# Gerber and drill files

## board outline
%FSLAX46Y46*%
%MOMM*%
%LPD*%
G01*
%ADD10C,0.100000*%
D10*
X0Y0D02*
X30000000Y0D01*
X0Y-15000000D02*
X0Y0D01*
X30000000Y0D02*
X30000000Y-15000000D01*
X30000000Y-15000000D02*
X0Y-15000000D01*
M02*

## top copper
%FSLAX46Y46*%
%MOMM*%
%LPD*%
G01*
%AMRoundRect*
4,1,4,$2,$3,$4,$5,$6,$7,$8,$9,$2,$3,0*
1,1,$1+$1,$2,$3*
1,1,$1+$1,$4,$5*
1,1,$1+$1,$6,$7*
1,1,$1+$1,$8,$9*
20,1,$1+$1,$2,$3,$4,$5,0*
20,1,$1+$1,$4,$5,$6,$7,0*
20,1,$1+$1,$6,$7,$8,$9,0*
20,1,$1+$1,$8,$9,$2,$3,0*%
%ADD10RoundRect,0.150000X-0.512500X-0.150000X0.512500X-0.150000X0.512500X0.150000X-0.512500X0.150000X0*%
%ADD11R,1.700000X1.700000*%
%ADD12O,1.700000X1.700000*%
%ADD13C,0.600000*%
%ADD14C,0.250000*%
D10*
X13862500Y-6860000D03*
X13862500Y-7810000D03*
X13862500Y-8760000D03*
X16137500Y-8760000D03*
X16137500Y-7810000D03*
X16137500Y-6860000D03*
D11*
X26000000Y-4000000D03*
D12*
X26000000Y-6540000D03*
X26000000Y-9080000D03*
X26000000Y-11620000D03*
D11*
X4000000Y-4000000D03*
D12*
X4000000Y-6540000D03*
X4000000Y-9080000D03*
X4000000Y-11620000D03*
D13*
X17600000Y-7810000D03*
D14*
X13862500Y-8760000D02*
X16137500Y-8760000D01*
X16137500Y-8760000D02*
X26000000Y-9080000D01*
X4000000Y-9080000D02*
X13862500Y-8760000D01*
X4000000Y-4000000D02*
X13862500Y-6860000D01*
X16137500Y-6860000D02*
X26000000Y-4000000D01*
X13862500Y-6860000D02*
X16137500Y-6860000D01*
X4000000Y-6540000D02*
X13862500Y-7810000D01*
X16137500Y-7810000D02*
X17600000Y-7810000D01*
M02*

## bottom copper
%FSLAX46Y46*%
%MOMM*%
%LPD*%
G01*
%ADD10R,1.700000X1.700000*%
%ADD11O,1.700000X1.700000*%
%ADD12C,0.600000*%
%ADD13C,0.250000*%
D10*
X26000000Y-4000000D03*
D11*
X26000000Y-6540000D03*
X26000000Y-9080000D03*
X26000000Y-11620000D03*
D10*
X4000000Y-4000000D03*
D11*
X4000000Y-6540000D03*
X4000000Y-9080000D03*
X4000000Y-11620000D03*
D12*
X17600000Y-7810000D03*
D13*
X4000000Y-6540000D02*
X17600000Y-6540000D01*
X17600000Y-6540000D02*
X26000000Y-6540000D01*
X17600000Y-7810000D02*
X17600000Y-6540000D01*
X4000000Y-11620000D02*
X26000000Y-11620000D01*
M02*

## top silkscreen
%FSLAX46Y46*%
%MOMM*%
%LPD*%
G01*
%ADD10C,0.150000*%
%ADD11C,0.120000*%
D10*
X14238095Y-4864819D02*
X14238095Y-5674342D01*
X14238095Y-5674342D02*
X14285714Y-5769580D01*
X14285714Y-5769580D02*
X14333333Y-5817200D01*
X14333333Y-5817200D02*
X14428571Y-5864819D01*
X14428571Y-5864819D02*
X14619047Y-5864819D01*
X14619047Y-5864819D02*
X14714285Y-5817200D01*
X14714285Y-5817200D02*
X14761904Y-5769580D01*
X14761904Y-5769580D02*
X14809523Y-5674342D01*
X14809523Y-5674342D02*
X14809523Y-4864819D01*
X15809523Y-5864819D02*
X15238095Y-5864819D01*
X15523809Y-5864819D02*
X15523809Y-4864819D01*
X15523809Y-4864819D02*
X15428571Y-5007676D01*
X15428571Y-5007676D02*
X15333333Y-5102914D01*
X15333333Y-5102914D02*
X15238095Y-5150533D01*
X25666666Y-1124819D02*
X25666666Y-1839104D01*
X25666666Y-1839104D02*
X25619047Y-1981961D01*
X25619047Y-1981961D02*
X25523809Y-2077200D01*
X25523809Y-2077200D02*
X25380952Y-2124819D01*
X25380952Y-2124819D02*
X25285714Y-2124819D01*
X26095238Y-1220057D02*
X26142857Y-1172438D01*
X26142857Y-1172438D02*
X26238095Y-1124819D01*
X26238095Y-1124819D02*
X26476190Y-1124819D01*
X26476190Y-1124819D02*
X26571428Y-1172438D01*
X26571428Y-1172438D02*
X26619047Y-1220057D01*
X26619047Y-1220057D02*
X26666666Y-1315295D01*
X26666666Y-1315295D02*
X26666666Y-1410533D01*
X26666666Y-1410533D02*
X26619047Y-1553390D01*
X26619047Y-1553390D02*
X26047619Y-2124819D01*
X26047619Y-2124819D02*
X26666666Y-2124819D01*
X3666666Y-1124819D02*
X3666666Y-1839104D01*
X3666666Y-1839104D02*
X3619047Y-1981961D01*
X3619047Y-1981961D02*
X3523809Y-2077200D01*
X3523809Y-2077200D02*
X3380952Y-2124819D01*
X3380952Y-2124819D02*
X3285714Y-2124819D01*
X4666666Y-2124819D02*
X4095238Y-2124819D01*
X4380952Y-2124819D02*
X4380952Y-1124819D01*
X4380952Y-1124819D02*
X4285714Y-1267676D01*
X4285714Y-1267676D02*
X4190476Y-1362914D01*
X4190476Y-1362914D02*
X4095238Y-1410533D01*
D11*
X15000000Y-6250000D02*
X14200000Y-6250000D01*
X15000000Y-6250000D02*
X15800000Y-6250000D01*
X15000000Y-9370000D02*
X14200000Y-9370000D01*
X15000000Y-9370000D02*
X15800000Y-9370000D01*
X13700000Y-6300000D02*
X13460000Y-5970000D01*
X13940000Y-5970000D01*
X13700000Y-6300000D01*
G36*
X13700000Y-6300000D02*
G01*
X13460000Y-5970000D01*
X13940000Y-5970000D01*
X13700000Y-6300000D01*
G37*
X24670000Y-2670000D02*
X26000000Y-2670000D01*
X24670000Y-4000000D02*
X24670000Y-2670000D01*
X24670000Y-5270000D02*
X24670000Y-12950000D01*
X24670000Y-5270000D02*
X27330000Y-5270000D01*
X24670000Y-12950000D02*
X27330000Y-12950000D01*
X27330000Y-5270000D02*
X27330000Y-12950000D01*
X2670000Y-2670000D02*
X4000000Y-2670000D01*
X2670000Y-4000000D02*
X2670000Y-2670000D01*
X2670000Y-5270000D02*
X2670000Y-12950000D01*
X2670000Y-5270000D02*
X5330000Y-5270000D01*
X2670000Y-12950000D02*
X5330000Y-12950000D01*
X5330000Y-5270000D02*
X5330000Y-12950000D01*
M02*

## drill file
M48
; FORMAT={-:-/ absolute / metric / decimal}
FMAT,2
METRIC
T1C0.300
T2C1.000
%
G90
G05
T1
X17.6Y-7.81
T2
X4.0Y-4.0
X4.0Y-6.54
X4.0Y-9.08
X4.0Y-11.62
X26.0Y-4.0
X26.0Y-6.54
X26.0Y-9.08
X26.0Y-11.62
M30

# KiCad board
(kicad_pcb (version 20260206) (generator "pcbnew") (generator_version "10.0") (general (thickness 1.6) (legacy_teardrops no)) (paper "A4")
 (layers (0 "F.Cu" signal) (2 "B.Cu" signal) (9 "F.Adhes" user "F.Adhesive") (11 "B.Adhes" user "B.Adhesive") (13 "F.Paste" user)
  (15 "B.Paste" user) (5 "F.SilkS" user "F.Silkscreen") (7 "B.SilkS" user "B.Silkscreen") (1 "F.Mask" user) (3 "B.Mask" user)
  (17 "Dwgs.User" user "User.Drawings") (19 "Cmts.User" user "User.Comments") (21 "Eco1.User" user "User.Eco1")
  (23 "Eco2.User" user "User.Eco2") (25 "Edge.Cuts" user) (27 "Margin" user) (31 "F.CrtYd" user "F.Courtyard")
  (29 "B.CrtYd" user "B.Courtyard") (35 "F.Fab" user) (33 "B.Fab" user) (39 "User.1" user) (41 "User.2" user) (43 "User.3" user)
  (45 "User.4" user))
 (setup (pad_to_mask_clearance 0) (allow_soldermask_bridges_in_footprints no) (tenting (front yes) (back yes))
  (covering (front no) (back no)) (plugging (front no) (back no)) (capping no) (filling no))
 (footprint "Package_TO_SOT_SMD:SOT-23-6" (layer "F.Cu") (at 15 7.81)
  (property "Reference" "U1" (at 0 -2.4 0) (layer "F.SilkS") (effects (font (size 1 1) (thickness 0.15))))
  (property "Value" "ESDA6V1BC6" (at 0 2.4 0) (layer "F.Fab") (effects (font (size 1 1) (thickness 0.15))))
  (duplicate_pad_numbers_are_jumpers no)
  (fp_line (start 0 -1.56) (end -0.8 -1.56) (stroke (width 0.12) (type solid)) (layer "F.SilkS"))
  (fp_line (start 0 -1.56) (end 0.8 -1.56) (stroke (width 0.12) (type solid)) (layer "F.SilkS"))
  (fp_line (start 0 1.56) (end -0.8 1.56) (stroke (width 0.12) (type solid)) (layer "F.SilkS"))
  (fp_line (start 0 1.56) (end 0.8 1.56) (stroke (width 0.12) (type solid)) (layer "F.SilkS"))
  (fp_poly
   (pts (xy -1.3 -1.51) (xy -1.54 -1.84) (xy -1.06 -1.84) (xy -1.3 -1.51)) (stroke (width 0.12) (type solid)) (fill yes) (layer "F.SilkS"))
  (pad "1" smd roundrect (at -1.1375 -0.95) (size 1.325 0.6) (layers "F.Cu" "F.Mask" "F.Paste") (roundrect_rratio 0.25) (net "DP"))
  (pad "2" smd roundrect (at -1.1375 0) (size 1.325 0.6) (layers "F.Cu" "F.Mask" "F.Paste") (roundrect_rratio 0.25) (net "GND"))
  (pad "3" smd roundrect (at -1.1375 0.95) (size 1.325 0.6) (layers "F.Cu" "F.Mask" "F.Paste") (roundrect_rratio 0.25) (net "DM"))
  (pad "4" smd roundrect (at 1.1375 0.95) (size 1.325 0.6) (layers "F.Cu" "F.Mask" "F.Paste") (roundrect_rratio 0.25) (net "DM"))
  (pad "5" smd roundrect (at 1.1375 0) (size 1.325 0.6) (layers "F.Cu" "F.Mask" "F.Paste") (roundrect_rratio 0.25) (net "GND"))
  (pad "6" smd roundrect (at 1.1375 -0.95) (size 1.325 0.6) (layers "F.Cu" "F.Mask" "F.Paste") (roundrect_rratio 0.25) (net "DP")))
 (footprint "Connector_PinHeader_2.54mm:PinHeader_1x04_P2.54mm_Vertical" (layer "F.Cu") (at 26 4)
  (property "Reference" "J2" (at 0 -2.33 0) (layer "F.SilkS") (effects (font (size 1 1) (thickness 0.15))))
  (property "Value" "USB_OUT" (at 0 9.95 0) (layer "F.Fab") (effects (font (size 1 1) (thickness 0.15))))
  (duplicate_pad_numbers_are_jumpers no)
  (fp_line (start -1.33 -1.33) (end 0 -1.33) (stroke (width 0.12) (type solid)) (layer "F.SilkS"))
  (fp_line (start -1.33 0) (end -1.33 -1.33) (stroke (width 0.12) (type solid)) (layer "F.SilkS"))
  (fp_line (start -1.33 1.27) (end -1.33 8.95) (stroke (width 0.12) (type solid)) (layer "F.SilkS"))
  (fp_line (start -1.33 1.27) (end 1.33 1.27) (stroke (width 0.12) (type solid)) (layer "F.SilkS"))
  (fp_line (start -1.33 8.95) (end 1.33 8.95) (stroke (width 0.12) (type solid)) (layer "F.SilkS"))
  (fp_line (start 1.33 1.27) (end 1.33 8.95) (stroke (width 0.12) (type solid)) (layer "F.SilkS"))
  (pad "1" thru_hole rect (at 0 0) (size 1.7 1.7) (drill 1) (layers "*.Cu" "*.Mask") (remove_unused_layers no) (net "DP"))
  (pad "2" thru_hole oval (at 0 2.54) (size 1.7 1.7) (drill 1) (layers "*.Cu" "*.Mask") (remove_unused_layers no) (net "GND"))
  (pad "3" thru_hole oval (at 0 5.08) (size 1.7 1.7) (drill 1) (layers "*.Cu" "*.Mask") (remove_unused_layers no) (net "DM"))
  (pad "4" thru_hole oval (at 0 7.62) (size 1.7 1.7) (drill 1) (layers "*.Cu" "*.Mask") (remove_unused_layers no) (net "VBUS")))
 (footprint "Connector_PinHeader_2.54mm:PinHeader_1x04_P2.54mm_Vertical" (layer "F.Cu") (at 4 4)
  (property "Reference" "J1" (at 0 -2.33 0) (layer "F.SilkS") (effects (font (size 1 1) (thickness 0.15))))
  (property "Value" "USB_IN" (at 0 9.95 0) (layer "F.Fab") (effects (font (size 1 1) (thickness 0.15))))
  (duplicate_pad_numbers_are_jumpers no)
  (fp_line (start -1.33 -1.33) (end 0 -1.33) (stroke (width 0.12) (type solid)) (layer "F.SilkS"))
  (fp_line (start -1.33 0) (end -1.33 -1.33) (stroke (width 0.12) (type solid)) (layer "F.SilkS"))
  (fp_line (start -1.33 1.27) (end -1.33 8.95) (stroke (width 0.12) (type solid)) (layer "F.SilkS"))
  (fp_line (start -1.33 1.27) (end 1.33 1.27) (stroke (width 0.12) (type solid)) (layer "F.SilkS"))
  (fp_line (start -1.33 8.95) (end 1.33 8.95) (stroke (width 0.12) (type solid)) (layer "F.SilkS"))
  (fp_line (start 1.33 1.27) (end 1.33 8.95) (stroke (width 0.12) (type solid)) (layer "F.SilkS"))
  (pad "1" thru_hole rect (at 0 0) (size 1.7 1.7) (drill 1) (layers "*.Cu" "*.Mask") (remove_unused_layers no) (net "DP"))
  (pad "2" thru_hole oval (at 0 2.54) (size 1.7 1.7) (drill 1) (layers "*.Cu" "*.Mask") (remove_unused_layers no) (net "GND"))
  (pad "3" thru_hole oval (at 0 5.08) (size 1.7 1.7) (drill 1) (layers "*.Cu" "*.Mask") (remove_unused_layers no) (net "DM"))
  (pad "4" thru_hole oval (at 0 7.62) (size 1.7 1.7) (drill 1) (layers "*.Cu" "*.Mask") (remove_unused_layers no) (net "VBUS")))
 (gr_line (start 0 0) (end 30 0) (stroke (width 0.1) (type default)) (layer "Edge.Cuts"))
 (gr_line (start 0 15) (end 0 0) (stroke (width 0.1) (type default)) (layer "Edge.Cuts"))
 (gr_line (start 30 0) (end 30 15) (stroke (width 0.1) (type default)) (layer "Edge.Cuts"))
 (gr_line (start 30 15) (end 0 15) (stroke (width 0.1) (type default)) (layer "Edge.Cuts"))
 (segment (start 13.8625 8.76) (end 16.1375 8.76) (width 0.25) (layer "F.Cu") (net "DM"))
 (segment (start 16.1375 8.76) (end 26 9.08) (width 0.25) (layer "F.Cu") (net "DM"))
 (segment (start 4 9.08) (end 13.8625 8.76) (width 0.25) (layer "F.Cu") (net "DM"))
 (segment (start 4 4) (end 13.8625 6.86) (width 0.25) (layer "F.Cu") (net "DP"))
 (segment (start 16.1375 6.86) (end 26 4) (width 0.25) (layer "F.Cu") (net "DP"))
 (segment (start 13.8625 6.86) (end 16.1375 6.86) (width 0.25) (layer "F.Cu") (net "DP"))
 (segment (start 4 6.54) (end 13.8625 7.81) (width 0.25) (layer "F.Cu") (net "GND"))
 (segment (start 16.1375 7.81) (end 17.6 7.81) (width 0.25) (layer "F.Cu") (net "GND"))
 (via (at 17.6 7.81) (size 0.6) (drill 0.3) (layers "F.Cu" "B.Cu") (capping no) (covering (front no) (back no))
  (plugging (front no) (back no)) (filling no) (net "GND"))
 (segment (start 4 6.54) (end 17.6 6.54) (width 0.25) (layer "B.Cu") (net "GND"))
 (segment (start 17.6 6.54) (end 26 6.54) (width 0.25) (layer "B.Cu") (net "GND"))
 (segment (start 17.6 7.81) (end 17.6 6.54) (width 0.25) (layer "B.Cu") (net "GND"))
 (segment (start 4 11.62) (end 26 11.62) (width 0.25) (layer "B.Cu") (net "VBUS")))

